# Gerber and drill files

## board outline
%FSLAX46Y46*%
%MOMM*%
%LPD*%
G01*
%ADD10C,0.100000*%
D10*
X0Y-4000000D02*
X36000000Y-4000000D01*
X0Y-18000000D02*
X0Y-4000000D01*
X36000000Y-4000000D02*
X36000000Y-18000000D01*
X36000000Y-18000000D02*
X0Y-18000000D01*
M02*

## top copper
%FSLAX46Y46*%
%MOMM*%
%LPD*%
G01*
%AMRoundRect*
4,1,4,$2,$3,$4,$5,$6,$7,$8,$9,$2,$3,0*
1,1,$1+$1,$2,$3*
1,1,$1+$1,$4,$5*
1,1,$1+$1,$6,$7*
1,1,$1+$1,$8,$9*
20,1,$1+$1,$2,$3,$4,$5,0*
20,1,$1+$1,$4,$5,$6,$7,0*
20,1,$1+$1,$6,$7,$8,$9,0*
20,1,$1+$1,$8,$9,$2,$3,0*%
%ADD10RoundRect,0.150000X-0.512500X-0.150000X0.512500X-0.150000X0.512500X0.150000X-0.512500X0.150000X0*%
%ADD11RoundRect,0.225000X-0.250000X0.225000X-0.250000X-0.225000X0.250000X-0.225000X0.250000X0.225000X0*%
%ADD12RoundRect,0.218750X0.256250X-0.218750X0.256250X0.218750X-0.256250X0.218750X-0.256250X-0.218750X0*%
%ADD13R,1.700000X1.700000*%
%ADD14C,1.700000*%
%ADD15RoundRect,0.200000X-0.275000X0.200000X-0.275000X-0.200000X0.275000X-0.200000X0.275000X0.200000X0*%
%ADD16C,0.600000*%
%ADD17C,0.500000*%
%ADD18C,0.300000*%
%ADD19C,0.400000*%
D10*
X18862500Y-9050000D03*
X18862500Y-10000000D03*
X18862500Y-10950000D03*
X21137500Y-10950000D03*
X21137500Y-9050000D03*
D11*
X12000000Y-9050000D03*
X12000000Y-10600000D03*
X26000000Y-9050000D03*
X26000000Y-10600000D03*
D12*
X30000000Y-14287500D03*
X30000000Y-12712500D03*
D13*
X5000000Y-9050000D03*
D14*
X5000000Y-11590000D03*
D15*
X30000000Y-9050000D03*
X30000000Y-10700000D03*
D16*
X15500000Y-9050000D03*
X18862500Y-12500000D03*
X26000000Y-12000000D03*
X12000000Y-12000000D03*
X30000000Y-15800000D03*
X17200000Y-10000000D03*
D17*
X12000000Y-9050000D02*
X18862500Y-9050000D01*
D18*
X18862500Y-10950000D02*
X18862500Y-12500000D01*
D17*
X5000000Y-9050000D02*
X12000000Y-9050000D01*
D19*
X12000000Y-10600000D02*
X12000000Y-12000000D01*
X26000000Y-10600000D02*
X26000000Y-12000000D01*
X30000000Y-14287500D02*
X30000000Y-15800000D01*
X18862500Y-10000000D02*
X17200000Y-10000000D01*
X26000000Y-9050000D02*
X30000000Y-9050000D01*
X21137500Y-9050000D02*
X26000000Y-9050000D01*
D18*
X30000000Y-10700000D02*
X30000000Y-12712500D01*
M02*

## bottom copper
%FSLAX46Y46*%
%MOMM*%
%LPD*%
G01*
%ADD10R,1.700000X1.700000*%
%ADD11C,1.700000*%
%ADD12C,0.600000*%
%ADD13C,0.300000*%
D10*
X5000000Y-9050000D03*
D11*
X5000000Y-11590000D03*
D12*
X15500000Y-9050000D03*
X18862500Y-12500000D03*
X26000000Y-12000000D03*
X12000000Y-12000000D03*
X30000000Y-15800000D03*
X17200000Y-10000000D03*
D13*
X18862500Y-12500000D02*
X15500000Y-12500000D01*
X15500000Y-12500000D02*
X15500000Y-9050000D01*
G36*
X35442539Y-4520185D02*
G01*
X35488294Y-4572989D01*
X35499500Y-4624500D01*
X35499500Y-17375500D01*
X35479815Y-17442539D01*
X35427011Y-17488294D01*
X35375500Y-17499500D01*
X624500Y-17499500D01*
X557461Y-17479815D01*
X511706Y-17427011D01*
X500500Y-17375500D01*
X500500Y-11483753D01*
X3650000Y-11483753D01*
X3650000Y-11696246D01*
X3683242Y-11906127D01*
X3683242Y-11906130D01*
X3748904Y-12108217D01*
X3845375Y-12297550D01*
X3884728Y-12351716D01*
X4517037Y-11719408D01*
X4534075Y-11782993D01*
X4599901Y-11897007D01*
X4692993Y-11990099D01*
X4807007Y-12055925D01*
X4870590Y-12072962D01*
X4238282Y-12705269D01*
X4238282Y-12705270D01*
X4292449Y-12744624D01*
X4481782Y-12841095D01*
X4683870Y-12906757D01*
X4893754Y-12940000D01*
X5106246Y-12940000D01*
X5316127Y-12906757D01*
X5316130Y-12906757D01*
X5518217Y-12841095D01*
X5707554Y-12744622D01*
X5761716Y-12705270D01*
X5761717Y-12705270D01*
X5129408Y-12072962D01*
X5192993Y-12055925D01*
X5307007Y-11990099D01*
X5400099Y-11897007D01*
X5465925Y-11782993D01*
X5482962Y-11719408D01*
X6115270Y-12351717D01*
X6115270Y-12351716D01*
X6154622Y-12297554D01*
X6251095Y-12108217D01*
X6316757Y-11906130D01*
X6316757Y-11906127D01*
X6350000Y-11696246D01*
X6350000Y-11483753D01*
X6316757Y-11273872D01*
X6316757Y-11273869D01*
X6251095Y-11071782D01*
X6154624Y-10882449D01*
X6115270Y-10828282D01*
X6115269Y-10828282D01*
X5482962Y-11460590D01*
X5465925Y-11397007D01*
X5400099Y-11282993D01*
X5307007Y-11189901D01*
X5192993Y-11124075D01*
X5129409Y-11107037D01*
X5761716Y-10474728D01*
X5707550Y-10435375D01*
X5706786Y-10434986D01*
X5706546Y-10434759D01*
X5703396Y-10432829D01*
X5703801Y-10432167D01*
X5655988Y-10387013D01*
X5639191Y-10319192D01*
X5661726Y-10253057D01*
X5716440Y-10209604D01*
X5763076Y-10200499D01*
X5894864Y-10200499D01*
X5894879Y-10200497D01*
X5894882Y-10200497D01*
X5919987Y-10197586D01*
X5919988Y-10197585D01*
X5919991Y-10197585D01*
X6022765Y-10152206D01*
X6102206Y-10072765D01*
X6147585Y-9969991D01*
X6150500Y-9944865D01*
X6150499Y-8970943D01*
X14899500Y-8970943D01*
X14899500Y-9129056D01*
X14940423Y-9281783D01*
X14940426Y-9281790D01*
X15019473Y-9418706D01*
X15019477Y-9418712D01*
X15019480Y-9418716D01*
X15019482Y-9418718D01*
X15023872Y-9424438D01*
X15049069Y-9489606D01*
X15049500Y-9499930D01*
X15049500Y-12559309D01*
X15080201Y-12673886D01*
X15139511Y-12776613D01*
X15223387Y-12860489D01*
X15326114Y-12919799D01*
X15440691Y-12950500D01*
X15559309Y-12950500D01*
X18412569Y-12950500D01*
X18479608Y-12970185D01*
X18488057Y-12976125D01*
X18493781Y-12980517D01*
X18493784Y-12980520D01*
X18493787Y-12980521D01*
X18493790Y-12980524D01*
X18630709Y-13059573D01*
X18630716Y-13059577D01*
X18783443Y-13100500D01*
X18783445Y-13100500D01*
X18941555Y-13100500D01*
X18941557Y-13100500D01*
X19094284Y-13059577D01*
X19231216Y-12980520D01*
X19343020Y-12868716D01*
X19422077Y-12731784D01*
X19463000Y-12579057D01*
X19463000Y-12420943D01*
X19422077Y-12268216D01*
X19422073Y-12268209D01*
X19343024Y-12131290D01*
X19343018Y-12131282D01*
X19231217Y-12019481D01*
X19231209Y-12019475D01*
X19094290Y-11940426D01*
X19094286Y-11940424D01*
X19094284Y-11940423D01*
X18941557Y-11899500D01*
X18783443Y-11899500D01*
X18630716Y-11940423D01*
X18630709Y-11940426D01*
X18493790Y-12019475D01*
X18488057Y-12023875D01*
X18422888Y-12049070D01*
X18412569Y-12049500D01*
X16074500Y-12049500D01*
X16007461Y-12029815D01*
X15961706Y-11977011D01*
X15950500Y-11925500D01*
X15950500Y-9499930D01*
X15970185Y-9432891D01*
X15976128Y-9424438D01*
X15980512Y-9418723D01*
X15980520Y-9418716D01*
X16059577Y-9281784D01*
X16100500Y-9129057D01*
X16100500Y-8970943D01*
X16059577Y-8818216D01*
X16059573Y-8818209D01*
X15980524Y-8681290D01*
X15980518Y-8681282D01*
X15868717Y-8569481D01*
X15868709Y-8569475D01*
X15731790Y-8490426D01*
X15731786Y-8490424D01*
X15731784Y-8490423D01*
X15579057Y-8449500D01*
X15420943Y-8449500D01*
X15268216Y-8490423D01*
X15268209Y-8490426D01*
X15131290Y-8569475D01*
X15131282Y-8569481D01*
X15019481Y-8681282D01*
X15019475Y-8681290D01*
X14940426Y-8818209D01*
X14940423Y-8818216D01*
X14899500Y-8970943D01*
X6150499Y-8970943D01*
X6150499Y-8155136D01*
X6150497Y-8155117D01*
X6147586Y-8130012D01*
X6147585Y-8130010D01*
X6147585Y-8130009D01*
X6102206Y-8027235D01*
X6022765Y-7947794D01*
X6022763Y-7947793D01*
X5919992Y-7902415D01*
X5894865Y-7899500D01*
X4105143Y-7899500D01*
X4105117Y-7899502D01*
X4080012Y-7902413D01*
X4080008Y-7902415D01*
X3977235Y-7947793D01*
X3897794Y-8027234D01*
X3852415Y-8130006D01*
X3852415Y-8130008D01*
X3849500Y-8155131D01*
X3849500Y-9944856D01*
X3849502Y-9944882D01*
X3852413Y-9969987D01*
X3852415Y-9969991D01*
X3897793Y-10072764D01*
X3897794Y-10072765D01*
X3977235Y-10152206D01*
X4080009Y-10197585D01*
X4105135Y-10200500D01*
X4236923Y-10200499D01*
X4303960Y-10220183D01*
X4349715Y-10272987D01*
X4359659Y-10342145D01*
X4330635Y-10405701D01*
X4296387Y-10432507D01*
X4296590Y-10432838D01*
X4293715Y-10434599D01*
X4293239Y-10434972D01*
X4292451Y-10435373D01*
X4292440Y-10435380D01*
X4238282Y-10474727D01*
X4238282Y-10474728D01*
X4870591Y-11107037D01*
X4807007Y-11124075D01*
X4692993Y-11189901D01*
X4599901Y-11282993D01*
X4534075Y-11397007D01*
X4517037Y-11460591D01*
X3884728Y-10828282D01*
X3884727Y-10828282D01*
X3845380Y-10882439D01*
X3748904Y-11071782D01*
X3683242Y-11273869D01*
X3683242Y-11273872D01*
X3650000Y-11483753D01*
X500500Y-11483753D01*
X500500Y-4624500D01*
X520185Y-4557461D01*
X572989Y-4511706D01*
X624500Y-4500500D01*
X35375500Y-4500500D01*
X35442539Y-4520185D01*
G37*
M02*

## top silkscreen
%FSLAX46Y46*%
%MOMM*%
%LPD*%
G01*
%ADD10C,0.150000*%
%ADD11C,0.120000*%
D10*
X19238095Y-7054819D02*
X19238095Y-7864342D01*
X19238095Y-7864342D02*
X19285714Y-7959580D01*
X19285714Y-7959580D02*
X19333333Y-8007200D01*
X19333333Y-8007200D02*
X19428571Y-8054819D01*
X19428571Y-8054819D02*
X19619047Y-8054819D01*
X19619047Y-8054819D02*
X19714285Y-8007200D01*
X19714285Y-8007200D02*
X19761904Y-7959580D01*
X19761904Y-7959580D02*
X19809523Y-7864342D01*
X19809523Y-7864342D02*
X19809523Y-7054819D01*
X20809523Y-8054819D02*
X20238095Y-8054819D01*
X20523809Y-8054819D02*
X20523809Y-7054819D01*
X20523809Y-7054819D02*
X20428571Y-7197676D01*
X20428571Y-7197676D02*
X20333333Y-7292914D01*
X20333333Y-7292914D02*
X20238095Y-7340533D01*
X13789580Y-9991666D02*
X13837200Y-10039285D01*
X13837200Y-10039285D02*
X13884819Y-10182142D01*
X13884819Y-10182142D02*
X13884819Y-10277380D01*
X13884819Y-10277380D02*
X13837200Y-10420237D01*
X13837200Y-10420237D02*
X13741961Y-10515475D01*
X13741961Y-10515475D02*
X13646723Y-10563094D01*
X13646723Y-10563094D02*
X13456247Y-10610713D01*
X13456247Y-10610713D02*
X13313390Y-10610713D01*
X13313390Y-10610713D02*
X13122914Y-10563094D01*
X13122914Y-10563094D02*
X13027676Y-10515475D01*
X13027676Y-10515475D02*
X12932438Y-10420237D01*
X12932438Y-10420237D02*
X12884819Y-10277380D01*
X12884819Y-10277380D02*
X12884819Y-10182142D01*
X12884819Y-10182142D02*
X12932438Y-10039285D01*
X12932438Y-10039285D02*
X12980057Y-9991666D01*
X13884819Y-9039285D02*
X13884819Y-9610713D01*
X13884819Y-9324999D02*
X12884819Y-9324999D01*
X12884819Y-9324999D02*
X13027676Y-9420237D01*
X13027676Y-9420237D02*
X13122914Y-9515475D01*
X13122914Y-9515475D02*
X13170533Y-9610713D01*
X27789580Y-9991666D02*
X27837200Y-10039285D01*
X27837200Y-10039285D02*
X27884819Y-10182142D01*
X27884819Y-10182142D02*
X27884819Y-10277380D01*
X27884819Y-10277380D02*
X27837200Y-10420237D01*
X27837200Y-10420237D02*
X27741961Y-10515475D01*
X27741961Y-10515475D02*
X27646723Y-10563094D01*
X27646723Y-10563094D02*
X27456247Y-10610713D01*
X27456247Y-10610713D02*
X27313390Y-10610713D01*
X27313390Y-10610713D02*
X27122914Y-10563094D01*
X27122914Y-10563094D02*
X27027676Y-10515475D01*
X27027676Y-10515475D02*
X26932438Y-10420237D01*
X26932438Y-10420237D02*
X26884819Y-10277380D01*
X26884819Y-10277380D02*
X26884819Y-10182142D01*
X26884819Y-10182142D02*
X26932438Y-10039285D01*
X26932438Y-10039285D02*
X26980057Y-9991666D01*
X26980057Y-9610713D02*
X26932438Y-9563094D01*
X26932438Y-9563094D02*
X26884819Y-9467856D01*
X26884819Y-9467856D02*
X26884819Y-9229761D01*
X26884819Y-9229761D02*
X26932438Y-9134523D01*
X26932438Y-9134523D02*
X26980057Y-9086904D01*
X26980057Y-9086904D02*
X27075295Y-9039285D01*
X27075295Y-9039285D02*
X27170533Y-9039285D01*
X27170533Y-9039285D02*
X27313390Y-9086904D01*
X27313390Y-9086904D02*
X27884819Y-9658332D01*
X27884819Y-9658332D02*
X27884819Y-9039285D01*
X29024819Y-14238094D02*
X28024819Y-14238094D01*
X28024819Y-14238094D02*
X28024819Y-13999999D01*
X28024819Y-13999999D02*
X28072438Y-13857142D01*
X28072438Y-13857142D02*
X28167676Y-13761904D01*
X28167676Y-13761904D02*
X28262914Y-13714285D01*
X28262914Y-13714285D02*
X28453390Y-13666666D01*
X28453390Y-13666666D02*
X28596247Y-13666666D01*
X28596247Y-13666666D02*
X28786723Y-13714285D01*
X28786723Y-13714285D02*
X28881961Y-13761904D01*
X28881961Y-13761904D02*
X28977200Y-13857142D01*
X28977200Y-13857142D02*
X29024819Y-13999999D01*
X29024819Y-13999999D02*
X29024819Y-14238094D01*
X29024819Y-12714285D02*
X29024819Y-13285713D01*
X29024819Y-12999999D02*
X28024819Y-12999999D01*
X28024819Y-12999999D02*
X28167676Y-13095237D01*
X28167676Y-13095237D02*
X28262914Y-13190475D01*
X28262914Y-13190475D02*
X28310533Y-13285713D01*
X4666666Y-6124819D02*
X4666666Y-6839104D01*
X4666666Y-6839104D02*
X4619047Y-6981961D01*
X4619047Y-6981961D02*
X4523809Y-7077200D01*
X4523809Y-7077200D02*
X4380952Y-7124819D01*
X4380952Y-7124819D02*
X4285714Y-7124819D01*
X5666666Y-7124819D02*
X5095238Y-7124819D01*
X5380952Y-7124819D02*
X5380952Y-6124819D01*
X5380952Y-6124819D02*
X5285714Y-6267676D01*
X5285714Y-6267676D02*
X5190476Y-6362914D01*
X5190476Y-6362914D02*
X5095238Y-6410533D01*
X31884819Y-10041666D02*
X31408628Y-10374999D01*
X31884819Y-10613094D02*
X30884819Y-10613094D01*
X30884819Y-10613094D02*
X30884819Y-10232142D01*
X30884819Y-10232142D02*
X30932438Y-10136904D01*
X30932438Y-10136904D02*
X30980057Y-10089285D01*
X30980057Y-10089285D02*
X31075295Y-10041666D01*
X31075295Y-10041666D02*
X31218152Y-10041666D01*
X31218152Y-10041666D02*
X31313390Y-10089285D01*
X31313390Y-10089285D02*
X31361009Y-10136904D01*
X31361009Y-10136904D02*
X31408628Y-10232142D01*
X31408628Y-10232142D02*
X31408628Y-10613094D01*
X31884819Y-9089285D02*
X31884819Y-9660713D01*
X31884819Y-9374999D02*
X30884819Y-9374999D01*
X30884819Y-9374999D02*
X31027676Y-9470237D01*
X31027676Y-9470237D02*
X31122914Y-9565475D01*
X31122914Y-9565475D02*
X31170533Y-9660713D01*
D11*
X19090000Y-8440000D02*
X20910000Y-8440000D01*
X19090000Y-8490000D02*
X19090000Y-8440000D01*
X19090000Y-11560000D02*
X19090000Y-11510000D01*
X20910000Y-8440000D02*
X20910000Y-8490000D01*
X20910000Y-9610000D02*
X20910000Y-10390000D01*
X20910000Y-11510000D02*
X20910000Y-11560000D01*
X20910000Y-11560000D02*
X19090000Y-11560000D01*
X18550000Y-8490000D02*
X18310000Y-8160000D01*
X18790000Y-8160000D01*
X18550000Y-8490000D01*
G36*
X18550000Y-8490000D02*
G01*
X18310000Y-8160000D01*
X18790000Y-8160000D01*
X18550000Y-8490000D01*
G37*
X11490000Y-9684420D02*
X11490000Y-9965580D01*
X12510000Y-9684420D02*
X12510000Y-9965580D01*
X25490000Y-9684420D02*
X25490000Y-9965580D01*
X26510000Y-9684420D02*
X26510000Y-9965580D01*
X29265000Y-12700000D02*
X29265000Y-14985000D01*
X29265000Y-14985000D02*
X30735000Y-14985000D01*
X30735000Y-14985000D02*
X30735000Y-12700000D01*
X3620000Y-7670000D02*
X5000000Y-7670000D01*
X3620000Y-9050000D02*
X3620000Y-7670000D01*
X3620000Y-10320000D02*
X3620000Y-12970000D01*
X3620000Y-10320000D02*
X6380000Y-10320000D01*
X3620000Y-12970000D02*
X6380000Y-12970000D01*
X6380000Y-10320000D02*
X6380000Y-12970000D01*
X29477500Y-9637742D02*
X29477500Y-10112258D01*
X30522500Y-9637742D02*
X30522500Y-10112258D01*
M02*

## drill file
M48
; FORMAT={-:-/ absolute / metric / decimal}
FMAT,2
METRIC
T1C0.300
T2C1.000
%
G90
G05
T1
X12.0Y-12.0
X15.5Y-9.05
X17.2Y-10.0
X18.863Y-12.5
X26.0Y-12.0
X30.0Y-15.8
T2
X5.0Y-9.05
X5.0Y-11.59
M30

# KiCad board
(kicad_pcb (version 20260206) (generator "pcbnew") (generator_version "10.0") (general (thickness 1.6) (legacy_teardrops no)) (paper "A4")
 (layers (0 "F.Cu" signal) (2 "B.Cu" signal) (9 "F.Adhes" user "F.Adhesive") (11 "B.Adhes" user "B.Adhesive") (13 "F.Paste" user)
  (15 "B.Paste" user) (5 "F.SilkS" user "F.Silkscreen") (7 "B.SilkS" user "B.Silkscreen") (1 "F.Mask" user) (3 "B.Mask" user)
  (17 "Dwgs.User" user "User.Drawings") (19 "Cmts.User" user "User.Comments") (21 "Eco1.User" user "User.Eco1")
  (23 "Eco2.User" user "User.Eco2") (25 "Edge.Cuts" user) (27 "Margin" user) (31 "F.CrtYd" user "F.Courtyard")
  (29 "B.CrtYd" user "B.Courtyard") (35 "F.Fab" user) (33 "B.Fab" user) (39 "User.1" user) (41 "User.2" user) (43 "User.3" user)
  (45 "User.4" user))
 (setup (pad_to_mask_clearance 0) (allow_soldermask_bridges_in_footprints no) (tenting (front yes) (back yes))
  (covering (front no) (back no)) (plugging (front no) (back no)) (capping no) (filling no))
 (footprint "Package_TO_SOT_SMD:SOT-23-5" (layer "F.Cu") (at 20 10)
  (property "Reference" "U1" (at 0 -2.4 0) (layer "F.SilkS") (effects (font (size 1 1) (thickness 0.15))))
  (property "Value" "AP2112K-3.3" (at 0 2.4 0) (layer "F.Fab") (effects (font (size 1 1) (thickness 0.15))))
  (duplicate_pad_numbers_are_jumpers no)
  (fp_line (start -0.91 -1.56) (end 0.91 -1.56) (stroke (width 0.12) (type solid)) (layer "F.SilkS"))
  (fp_line (start -0.91 -1.51) (end -0.91 -1.56) (stroke (width 0.12) (type solid)) (layer "F.SilkS"))
  (fp_line (start -0.91 1.56) (end -0.91 1.51) (stroke (width 0.12) (type solid)) (layer "F.SilkS"))
  (fp_line (start 0.91 -1.56) (end 0.91 -1.51) (stroke (width 0.12) (type solid)) (layer "F.SilkS"))
  (fp_line (start 0.91 -0.39) (end 0.91 0.39) (stroke (width 0.12) (type solid)) (layer "F.SilkS"))
  (fp_line (start 0.91 1.51) (end 0.91 1.56) (stroke (width 0.12) (type solid)) (layer "F.SilkS"))
  (fp_line (start 0.91 1.56) (end -0.91 1.56) (stroke (width 0.12) (type solid)) (layer "F.SilkS"))
  (fp_poly (pts (xy -1.45 -1.51) (xy -1.69 -1.84) (xy -1.21 -1.84)) (stroke (width 0.12) (type solid)) (fill yes) (layer "F.SilkS"))
  (pad "1" smd roundrect (at -1.1375 -0.95) (size 1.325 0.6) (layers "F.Cu" "F.Mask" "F.Paste") (roundrect_rratio 0.25) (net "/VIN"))
  (pad "2" smd roundrect (at -1.1375 0) (size 1.325 0.6) (layers "F.Cu" "F.Mask" "F.Paste") (roundrect_rratio 0.25) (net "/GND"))
  (pad "3" smd roundrect (at -1.1375 0.95) (size 1.325 0.6) (layers "F.Cu" "F.Mask" "F.Paste") (roundrect_rratio 0.25) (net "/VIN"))
  (pad "4" smd roundrect (at 1.1375 0.95) (size 1.325 0.6) (layers "F.Cu" "F.Mask" "F.Paste") (roundrect_rratio 0.25)
   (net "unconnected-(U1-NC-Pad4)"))
  (pad "5" smd roundrect (at 1.1375 -0.95) (size 1.325 0.6) (layers "F.Cu" "F.Mask" "F.Paste") (roundrect_rratio 0.25) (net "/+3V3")))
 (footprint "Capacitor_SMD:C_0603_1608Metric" (layer "F.Cu") (at 12 9.825 -90)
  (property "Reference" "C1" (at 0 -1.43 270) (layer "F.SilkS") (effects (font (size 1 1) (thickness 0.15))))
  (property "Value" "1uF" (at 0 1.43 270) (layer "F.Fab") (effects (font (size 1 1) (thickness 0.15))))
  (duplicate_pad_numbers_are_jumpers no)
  (fp_line (start -0.14058 0.51) (end 0.14058 0.51) (stroke (width 0.12) (type solid)) (layer "F.SilkS"))
  (fp_line (start -0.14058 -0.51) (end 0.14058 -0.51) (stroke (width 0.12) (type solid)) (layer "F.SilkS"))
  (pad "1" smd roundrect (at -0.775 0 270) (size 0.9 0.95) (layers "F.Cu" "F.Mask" "F.Paste") (roundrect_rratio 0.25) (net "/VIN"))
  (pad "2" smd roundrect (at 0.775 0 270) (size 0.9 0.95) (layers "F.Cu" "F.Mask" "F.Paste") (roundrect_rratio 0.25) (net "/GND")))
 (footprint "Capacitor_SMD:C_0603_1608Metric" (layer "F.Cu") (at 26 9.825 -90)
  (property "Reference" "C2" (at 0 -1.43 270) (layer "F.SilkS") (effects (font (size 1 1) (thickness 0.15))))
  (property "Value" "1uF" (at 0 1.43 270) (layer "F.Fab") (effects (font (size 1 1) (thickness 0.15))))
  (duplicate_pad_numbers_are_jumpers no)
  (fp_line (start -0.14058 0.51) (end 0.14058 0.51) (stroke (width 0.12) (type solid)) (layer "F.SilkS"))
  (fp_line (start -0.14058 -0.51) (end 0.14058 -0.51) (stroke (width 0.12) (type solid)) (layer "F.SilkS"))
  (pad "1" smd roundrect (at -0.775 0 270) (size 0.9 0.95) (layers "F.Cu" "F.Mask" "F.Paste") (roundrect_rratio 0.25) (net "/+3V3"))
  (pad "2" smd roundrect (at 0.775 0 270) (size 0.9 0.95) (layers "F.Cu" "F.Mask" "F.Paste") (roundrect_rratio 0.25) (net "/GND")))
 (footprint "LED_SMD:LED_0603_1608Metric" (layer "F.Cu") (at 30 13.5 90)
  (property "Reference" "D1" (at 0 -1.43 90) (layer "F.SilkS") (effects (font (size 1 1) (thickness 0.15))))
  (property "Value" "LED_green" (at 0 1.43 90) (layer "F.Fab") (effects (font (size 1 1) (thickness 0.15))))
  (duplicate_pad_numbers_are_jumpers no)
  (fp_line (start 0.8 -0.735) (end -1.485 -0.735) (stroke (width 0.12) (type solid)) (layer "F.SilkS"))
  (fp_line (start -1.485 -0.735) (end -1.485 0.735) (stroke (width 0.12) (type solid)) (layer "F.SilkS"))
  (fp_line (start -1.485 0.735) (end 0.8 0.735) (stroke (width 0.12) (type solid)) (layer "F.SilkS"))
  (pad "1" smd roundrect (at -0.7875 0 90) (size 0.875 0.95) (layers "F.Cu" "F.Mask" "F.Paste") (roundrect_rratio 0.25) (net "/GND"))
  (pad "2" smd roundrect (at 0.7875 0 90) (size 0.875 0.95) (layers "F.Cu" "F.Mask" "F.Paste") (roundrect_rratio 0.25) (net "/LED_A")))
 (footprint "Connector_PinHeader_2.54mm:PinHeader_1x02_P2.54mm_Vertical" (layer "F.Cu") (at 5 9.05)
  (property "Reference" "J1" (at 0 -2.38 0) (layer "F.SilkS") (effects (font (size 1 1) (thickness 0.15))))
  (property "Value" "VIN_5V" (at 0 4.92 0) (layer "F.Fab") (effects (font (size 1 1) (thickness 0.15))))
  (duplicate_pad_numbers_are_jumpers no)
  (fp_line (start -1.38 -1.38) (end 0 -1.38) (stroke (width 0.12) (type solid)) (layer "F.SilkS"))
  (fp_line (start -1.38 0) (end -1.38 -1.38) (stroke (width 0.12) (type solid)) (layer "F.SilkS"))
  (fp_line (start -1.38 1.27) (end -1.38 3.92) (stroke (width 0.12) (type solid)) (layer "F.SilkS"))
  (fp_line (start -1.38 1.27) (end 1.38 1.27) (stroke (width 0.12) (type solid)) (layer "F.SilkS"))
  (fp_line (start -1.38 3.92) (end 1.38 3.92) (stroke (width 0.12) (type solid)) (layer "F.SilkS"))
  (fp_line (start 1.38 1.27) (end 1.38 3.92) (stroke (width 0.12) (type solid)) (layer "F.SilkS"))
  (pad "1" thru_hole rect (at 0 0) (size 1.7 1.7) (drill 1) (layers "*.Cu" "*.Mask") (remove_unused_layers no) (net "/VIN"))
  (pad "2" thru_hole circle (at 0 2.54) (size 1.7 1.7) (drill 1) (layers "*.Cu" "*.Mask") (remove_unused_layers no) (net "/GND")))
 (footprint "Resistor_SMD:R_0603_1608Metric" (layer "F.Cu") (at 30 9.875 -90)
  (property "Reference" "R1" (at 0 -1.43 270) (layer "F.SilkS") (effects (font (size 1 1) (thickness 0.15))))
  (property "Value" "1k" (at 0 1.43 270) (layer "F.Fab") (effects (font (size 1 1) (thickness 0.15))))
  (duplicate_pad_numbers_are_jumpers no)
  (fp_line (start -0.237258 0.5225) (end 0.237258 0.5225) (stroke (width 0.12) (type solid)) (layer "F.SilkS"))
  (fp_line (start -0.237258 -0.5225) (end 0.237258 -0.5225) (stroke (width 0.12) (type solid)) (layer "F.SilkS"))
  (pad "1" smd roundrect (at -0.825 0 270) (size 0.8 0.95) (layers "F.Cu" "F.Mask" "F.Paste") (roundrect_rratio 0.25) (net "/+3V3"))
  (pad "2" smd roundrect (at 0.825 0 270) (size 0.8 0.95) (layers "F.Cu" "F.Mask" "F.Paste") (roundrect_rratio 0.25) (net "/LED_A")))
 (gr_line (start 0 4) (end 36 4) (stroke (width 0.1) (type default)) (layer "Edge.Cuts"))
 (gr_line (start 0 18) (end 0 4) (stroke (width 0.1) (type default)) (layer "Edge.Cuts"))
 (gr_line (start 36 4) (end 36 18) (stroke (width 0.1) (type default)) (layer "Edge.Cuts"))
 (gr_line (start 36 18) (end 0 18) (stroke (width 0.1) (type default)) (layer "Edge.Cuts"))
 (segment (start 12 9.05) (end 18.8625 9.05) (width 0.5) (layer "F.Cu") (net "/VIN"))
 (segment (start 18.8625 10.95) (end 18.8625 12.5) (width 0.3) (layer "F.Cu") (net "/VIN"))
 (segment (start 5 9.05) (end 12 9.05) (width 0.5) (layer "F.Cu") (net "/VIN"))
 (via (at 15.5 9.05) (size 0.6) (drill 0.3) (layers "F.Cu" "B.Cu") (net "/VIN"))
 (via (at 18.8625 12.5) (size 0.6) (drill 0.3) (layers "F.Cu" "B.Cu") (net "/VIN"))
 (segment (start 18.8625 12.5) (end 15.5 12.5) (width 0.3) (layer "B.Cu") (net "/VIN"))
 (segment (start 15.5 12.5) (end 15.5 9.05) (width 0.3) (layer "B.Cu") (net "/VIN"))
 (segment (start 12 10.6) (end 12 12) (width 0.4) (layer "F.Cu") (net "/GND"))
 (segment (start 26 10.6) (end 26 12) (width 0.4) (layer "F.Cu") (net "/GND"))
 (segment (start 30 14.2875) (end 30 15.8) (width 0.4) (layer "F.Cu") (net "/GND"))
 (segment (start 18.8625 10) (end 17.2 10) (width 0.4) (layer "F.Cu") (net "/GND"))
 (via (at 26 12) (size 0.6) (drill 0.3) (layers "F.Cu" "B.Cu") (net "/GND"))
 (via (at 12 12) (size 0.6) (drill 0.3) (layers "F.Cu" "B.Cu") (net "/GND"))
 (via (at 30 15.8) (size 0.6) (drill 0.3) (layers "F.Cu" "B.Cu") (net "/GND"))
 (via (at 17.2 10) (size 0.6) (drill 0.3) (layers "F.Cu" "B.Cu") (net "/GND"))
 (segment (start 26 9.05) (end 30 9.05) (width 0.4) (layer "F.Cu") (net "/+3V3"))
 (segment (start 21.1375 9.05) (end 26 9.05) (width 0.4) (layer "F.Cu") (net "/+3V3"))
 (segment (start 30 10.7) (end 30 12.7125) (width 0.3) (layer "F.Cu") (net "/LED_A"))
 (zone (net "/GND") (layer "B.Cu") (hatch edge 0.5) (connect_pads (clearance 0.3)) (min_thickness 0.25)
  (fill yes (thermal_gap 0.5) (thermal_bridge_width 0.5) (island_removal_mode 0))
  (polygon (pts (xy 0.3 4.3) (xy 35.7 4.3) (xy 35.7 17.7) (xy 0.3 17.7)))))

